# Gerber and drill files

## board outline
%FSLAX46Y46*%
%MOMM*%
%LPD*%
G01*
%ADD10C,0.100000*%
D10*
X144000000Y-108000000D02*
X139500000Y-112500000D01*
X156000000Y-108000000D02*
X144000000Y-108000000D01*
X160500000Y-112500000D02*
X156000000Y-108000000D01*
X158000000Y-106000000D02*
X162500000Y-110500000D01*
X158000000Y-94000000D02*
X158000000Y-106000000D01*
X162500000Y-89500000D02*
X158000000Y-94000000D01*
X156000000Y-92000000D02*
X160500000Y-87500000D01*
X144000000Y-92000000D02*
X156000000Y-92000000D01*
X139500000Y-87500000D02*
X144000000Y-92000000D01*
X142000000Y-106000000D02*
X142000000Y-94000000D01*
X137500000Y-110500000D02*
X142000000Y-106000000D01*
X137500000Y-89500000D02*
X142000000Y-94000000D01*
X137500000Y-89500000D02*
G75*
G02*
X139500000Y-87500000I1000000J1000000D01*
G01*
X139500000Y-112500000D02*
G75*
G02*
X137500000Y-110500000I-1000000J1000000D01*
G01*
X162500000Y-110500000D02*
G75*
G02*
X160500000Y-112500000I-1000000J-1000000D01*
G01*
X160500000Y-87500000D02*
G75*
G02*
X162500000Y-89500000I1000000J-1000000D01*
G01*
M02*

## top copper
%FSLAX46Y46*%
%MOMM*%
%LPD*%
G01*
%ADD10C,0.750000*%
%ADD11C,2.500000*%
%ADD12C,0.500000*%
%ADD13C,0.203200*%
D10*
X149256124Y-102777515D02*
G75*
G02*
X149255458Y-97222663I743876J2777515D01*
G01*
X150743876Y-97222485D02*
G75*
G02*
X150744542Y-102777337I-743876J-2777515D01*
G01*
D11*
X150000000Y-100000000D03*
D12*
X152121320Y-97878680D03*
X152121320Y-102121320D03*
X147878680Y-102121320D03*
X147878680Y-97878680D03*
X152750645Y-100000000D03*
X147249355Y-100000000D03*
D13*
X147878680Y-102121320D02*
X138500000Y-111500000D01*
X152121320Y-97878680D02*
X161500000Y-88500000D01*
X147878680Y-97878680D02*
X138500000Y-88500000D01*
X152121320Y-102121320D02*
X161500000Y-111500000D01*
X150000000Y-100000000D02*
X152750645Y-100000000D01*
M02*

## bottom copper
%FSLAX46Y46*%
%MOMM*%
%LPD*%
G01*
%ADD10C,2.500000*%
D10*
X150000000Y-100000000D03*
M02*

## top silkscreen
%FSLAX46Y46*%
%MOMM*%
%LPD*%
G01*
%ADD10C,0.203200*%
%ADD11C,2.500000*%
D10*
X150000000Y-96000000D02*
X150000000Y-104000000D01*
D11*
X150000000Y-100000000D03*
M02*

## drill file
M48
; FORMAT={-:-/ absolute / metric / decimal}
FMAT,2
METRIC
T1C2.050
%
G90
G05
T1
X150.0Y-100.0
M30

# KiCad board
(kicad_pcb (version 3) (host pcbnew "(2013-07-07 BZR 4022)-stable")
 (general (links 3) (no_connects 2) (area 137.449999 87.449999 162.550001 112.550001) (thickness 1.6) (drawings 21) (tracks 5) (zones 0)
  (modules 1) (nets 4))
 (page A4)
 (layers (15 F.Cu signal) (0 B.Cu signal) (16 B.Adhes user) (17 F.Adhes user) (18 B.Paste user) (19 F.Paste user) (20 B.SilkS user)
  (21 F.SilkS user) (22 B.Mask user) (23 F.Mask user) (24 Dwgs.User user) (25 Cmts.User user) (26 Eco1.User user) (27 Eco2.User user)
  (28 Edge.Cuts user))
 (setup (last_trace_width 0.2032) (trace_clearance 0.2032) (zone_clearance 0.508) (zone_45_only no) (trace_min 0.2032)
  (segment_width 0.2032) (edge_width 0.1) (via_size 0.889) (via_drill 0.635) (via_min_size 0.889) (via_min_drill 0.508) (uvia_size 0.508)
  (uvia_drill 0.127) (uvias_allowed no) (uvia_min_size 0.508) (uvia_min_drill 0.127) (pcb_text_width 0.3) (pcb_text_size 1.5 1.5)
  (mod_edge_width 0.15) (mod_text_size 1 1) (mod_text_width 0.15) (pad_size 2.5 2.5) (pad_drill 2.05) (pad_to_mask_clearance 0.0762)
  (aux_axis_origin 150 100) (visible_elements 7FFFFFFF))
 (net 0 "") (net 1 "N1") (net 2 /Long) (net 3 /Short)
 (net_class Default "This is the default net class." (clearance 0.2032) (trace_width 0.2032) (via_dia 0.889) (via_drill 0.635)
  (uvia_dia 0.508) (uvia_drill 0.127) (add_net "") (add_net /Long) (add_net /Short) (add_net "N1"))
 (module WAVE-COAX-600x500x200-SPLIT (layer F.Cu) (at 150 100 315) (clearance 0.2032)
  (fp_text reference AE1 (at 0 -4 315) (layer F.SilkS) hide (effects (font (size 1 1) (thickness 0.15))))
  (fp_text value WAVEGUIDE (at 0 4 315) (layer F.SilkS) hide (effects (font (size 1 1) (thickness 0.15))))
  (fp_arc (start 0 0) (end 1.438 2.49) (angle 150) (layer F.Cu) (width 0.75))
  (fp_arc (start 0 0) (end -1.438 -2.49) (angle 150) (layer F.Cu) (width 0.75))
  (pad C thru_hole circle (at 0 0 315) (size 2.5 2.5) (drill 2.05) (layers *.Cu *.Mask F.SilkS) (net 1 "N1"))
  (pad 1 smd circle (at 0 -3 315) (size 0.5 0.5) (layers F.Cu F.Paste F.Mask) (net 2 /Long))
  (pad 2 smd circle (at 3 0 315) (size 0.5 0.5) (layers F.Cu F.Paste F.Mask) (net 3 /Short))
  (pad 3 smd circle (at 0 3 315) (size 0.5 0.5) (layers F.Cu F.Paste F.Mask) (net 2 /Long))
  (pad 4 smd circle (at -3 0 315) (size 0.5 0.5) (layers F.Cu F.Paste F.Mask) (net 3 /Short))
  (pad 5 smd circle (at 1.945 -1.945 315) (size 0.5 0.5) (layers F.Cu F.Paste F.Mask) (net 1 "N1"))
  (pad 7 smd circle (at -1.945 1.945 315) (size 0.5 0.5) (layers F.Cu F.Paste F.Mask)))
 (gr_line (start 144 108) (end 139.5 112.5) (angle 90) (layer Edge.Cuts) (width 0.1))
 (gr_line (start 156 108) (end 144 108) (angle 90) (layer Edge.Cuts) (width 0.1))
 (gr_line (start 160.5 112.5) (end 156 108) (angle 90) (layer Edge.Cuts) (width 0.1))
 (gr_line (start 158 106) (end 162.5 110.5) (angle 90) (layer Edge.Cuts) (width 0.1))
 (gr_line (start 158 94) (end 158 106) (angle 90) (layer Edge.Cuts) (width 0.1))
 (gr_line (start 162.5 89.5) (end 158 94) (angle 90) (layer Edge.Cuts) (width 0.1))
 (gr_line (start 156 92) (end 160.5 87.5) (angle 90) (layer Edge.Cuts) (width 0.1))
 (gr_line (start 144 92) (end 156 92) (angle 90) (layer Edge.Cuts) (width 0.1))
 (gr_line (start 139.5 87.5) (end 144 92) (angle 90) (layer Edge.Cuts) (width 0.1))
 (gr_line (start 142 106) (end 142 94) (angle 90) (layer Edge.Cuts) (width 0.1))
 (gr_line (start 137.5 110.5) (end 142 106) (angle 90) (layer Edge.Cuts) (width 0.1))
 (gr_line (start 137.5 89.5) (end 142 94) (angle 90) (layer Edge.Cuts) (width 0.1))
 (gr_arc (start 138.5 88.5) (end 137.5 89.5) (angle 180) (layer Edge.Cuts) (width 0.1))
 (gr_arc (start 138.5 111.5) (end 139.5 112.5) (angle 180) (layer Edge.Cuts) (width 0.1))
 (gr_arc (start 161.5 111.5) (end 162.5 110.5) (angle 180) (layer Edge.Cuts) (width 0.1))
 (gr_arc (start 161.5 88.5) (end 160.5 87.5) (angle 180) (layer Edge.Cuts) (width 0.1))
 (gr_line (start 150 96) (end 150 104) (angle 90) (layer F.SilkS) (width 0.2032))
 (segment (start 147.87868 102.12132) (end 138.5 111.5) (width 0.2032) (layer F.Cu) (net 2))
 (segment (start 152.12132 97.87868) (end 161.5 88.5) (width 0.2032) (layer F.Cu) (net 2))
 (segment (start 147.87868 97.87868) (end 138.5 88.5) (width 0.2032) (layer F.Cu) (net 3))
 (segment (start 152.12132 102.12132) (end 161.5 111.5) (width 0.2032) (layer F.Cu) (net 3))
 (segment (start 150 100) (end 152.750645 100) (width 0.2032) (layer F.Cu) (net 1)))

